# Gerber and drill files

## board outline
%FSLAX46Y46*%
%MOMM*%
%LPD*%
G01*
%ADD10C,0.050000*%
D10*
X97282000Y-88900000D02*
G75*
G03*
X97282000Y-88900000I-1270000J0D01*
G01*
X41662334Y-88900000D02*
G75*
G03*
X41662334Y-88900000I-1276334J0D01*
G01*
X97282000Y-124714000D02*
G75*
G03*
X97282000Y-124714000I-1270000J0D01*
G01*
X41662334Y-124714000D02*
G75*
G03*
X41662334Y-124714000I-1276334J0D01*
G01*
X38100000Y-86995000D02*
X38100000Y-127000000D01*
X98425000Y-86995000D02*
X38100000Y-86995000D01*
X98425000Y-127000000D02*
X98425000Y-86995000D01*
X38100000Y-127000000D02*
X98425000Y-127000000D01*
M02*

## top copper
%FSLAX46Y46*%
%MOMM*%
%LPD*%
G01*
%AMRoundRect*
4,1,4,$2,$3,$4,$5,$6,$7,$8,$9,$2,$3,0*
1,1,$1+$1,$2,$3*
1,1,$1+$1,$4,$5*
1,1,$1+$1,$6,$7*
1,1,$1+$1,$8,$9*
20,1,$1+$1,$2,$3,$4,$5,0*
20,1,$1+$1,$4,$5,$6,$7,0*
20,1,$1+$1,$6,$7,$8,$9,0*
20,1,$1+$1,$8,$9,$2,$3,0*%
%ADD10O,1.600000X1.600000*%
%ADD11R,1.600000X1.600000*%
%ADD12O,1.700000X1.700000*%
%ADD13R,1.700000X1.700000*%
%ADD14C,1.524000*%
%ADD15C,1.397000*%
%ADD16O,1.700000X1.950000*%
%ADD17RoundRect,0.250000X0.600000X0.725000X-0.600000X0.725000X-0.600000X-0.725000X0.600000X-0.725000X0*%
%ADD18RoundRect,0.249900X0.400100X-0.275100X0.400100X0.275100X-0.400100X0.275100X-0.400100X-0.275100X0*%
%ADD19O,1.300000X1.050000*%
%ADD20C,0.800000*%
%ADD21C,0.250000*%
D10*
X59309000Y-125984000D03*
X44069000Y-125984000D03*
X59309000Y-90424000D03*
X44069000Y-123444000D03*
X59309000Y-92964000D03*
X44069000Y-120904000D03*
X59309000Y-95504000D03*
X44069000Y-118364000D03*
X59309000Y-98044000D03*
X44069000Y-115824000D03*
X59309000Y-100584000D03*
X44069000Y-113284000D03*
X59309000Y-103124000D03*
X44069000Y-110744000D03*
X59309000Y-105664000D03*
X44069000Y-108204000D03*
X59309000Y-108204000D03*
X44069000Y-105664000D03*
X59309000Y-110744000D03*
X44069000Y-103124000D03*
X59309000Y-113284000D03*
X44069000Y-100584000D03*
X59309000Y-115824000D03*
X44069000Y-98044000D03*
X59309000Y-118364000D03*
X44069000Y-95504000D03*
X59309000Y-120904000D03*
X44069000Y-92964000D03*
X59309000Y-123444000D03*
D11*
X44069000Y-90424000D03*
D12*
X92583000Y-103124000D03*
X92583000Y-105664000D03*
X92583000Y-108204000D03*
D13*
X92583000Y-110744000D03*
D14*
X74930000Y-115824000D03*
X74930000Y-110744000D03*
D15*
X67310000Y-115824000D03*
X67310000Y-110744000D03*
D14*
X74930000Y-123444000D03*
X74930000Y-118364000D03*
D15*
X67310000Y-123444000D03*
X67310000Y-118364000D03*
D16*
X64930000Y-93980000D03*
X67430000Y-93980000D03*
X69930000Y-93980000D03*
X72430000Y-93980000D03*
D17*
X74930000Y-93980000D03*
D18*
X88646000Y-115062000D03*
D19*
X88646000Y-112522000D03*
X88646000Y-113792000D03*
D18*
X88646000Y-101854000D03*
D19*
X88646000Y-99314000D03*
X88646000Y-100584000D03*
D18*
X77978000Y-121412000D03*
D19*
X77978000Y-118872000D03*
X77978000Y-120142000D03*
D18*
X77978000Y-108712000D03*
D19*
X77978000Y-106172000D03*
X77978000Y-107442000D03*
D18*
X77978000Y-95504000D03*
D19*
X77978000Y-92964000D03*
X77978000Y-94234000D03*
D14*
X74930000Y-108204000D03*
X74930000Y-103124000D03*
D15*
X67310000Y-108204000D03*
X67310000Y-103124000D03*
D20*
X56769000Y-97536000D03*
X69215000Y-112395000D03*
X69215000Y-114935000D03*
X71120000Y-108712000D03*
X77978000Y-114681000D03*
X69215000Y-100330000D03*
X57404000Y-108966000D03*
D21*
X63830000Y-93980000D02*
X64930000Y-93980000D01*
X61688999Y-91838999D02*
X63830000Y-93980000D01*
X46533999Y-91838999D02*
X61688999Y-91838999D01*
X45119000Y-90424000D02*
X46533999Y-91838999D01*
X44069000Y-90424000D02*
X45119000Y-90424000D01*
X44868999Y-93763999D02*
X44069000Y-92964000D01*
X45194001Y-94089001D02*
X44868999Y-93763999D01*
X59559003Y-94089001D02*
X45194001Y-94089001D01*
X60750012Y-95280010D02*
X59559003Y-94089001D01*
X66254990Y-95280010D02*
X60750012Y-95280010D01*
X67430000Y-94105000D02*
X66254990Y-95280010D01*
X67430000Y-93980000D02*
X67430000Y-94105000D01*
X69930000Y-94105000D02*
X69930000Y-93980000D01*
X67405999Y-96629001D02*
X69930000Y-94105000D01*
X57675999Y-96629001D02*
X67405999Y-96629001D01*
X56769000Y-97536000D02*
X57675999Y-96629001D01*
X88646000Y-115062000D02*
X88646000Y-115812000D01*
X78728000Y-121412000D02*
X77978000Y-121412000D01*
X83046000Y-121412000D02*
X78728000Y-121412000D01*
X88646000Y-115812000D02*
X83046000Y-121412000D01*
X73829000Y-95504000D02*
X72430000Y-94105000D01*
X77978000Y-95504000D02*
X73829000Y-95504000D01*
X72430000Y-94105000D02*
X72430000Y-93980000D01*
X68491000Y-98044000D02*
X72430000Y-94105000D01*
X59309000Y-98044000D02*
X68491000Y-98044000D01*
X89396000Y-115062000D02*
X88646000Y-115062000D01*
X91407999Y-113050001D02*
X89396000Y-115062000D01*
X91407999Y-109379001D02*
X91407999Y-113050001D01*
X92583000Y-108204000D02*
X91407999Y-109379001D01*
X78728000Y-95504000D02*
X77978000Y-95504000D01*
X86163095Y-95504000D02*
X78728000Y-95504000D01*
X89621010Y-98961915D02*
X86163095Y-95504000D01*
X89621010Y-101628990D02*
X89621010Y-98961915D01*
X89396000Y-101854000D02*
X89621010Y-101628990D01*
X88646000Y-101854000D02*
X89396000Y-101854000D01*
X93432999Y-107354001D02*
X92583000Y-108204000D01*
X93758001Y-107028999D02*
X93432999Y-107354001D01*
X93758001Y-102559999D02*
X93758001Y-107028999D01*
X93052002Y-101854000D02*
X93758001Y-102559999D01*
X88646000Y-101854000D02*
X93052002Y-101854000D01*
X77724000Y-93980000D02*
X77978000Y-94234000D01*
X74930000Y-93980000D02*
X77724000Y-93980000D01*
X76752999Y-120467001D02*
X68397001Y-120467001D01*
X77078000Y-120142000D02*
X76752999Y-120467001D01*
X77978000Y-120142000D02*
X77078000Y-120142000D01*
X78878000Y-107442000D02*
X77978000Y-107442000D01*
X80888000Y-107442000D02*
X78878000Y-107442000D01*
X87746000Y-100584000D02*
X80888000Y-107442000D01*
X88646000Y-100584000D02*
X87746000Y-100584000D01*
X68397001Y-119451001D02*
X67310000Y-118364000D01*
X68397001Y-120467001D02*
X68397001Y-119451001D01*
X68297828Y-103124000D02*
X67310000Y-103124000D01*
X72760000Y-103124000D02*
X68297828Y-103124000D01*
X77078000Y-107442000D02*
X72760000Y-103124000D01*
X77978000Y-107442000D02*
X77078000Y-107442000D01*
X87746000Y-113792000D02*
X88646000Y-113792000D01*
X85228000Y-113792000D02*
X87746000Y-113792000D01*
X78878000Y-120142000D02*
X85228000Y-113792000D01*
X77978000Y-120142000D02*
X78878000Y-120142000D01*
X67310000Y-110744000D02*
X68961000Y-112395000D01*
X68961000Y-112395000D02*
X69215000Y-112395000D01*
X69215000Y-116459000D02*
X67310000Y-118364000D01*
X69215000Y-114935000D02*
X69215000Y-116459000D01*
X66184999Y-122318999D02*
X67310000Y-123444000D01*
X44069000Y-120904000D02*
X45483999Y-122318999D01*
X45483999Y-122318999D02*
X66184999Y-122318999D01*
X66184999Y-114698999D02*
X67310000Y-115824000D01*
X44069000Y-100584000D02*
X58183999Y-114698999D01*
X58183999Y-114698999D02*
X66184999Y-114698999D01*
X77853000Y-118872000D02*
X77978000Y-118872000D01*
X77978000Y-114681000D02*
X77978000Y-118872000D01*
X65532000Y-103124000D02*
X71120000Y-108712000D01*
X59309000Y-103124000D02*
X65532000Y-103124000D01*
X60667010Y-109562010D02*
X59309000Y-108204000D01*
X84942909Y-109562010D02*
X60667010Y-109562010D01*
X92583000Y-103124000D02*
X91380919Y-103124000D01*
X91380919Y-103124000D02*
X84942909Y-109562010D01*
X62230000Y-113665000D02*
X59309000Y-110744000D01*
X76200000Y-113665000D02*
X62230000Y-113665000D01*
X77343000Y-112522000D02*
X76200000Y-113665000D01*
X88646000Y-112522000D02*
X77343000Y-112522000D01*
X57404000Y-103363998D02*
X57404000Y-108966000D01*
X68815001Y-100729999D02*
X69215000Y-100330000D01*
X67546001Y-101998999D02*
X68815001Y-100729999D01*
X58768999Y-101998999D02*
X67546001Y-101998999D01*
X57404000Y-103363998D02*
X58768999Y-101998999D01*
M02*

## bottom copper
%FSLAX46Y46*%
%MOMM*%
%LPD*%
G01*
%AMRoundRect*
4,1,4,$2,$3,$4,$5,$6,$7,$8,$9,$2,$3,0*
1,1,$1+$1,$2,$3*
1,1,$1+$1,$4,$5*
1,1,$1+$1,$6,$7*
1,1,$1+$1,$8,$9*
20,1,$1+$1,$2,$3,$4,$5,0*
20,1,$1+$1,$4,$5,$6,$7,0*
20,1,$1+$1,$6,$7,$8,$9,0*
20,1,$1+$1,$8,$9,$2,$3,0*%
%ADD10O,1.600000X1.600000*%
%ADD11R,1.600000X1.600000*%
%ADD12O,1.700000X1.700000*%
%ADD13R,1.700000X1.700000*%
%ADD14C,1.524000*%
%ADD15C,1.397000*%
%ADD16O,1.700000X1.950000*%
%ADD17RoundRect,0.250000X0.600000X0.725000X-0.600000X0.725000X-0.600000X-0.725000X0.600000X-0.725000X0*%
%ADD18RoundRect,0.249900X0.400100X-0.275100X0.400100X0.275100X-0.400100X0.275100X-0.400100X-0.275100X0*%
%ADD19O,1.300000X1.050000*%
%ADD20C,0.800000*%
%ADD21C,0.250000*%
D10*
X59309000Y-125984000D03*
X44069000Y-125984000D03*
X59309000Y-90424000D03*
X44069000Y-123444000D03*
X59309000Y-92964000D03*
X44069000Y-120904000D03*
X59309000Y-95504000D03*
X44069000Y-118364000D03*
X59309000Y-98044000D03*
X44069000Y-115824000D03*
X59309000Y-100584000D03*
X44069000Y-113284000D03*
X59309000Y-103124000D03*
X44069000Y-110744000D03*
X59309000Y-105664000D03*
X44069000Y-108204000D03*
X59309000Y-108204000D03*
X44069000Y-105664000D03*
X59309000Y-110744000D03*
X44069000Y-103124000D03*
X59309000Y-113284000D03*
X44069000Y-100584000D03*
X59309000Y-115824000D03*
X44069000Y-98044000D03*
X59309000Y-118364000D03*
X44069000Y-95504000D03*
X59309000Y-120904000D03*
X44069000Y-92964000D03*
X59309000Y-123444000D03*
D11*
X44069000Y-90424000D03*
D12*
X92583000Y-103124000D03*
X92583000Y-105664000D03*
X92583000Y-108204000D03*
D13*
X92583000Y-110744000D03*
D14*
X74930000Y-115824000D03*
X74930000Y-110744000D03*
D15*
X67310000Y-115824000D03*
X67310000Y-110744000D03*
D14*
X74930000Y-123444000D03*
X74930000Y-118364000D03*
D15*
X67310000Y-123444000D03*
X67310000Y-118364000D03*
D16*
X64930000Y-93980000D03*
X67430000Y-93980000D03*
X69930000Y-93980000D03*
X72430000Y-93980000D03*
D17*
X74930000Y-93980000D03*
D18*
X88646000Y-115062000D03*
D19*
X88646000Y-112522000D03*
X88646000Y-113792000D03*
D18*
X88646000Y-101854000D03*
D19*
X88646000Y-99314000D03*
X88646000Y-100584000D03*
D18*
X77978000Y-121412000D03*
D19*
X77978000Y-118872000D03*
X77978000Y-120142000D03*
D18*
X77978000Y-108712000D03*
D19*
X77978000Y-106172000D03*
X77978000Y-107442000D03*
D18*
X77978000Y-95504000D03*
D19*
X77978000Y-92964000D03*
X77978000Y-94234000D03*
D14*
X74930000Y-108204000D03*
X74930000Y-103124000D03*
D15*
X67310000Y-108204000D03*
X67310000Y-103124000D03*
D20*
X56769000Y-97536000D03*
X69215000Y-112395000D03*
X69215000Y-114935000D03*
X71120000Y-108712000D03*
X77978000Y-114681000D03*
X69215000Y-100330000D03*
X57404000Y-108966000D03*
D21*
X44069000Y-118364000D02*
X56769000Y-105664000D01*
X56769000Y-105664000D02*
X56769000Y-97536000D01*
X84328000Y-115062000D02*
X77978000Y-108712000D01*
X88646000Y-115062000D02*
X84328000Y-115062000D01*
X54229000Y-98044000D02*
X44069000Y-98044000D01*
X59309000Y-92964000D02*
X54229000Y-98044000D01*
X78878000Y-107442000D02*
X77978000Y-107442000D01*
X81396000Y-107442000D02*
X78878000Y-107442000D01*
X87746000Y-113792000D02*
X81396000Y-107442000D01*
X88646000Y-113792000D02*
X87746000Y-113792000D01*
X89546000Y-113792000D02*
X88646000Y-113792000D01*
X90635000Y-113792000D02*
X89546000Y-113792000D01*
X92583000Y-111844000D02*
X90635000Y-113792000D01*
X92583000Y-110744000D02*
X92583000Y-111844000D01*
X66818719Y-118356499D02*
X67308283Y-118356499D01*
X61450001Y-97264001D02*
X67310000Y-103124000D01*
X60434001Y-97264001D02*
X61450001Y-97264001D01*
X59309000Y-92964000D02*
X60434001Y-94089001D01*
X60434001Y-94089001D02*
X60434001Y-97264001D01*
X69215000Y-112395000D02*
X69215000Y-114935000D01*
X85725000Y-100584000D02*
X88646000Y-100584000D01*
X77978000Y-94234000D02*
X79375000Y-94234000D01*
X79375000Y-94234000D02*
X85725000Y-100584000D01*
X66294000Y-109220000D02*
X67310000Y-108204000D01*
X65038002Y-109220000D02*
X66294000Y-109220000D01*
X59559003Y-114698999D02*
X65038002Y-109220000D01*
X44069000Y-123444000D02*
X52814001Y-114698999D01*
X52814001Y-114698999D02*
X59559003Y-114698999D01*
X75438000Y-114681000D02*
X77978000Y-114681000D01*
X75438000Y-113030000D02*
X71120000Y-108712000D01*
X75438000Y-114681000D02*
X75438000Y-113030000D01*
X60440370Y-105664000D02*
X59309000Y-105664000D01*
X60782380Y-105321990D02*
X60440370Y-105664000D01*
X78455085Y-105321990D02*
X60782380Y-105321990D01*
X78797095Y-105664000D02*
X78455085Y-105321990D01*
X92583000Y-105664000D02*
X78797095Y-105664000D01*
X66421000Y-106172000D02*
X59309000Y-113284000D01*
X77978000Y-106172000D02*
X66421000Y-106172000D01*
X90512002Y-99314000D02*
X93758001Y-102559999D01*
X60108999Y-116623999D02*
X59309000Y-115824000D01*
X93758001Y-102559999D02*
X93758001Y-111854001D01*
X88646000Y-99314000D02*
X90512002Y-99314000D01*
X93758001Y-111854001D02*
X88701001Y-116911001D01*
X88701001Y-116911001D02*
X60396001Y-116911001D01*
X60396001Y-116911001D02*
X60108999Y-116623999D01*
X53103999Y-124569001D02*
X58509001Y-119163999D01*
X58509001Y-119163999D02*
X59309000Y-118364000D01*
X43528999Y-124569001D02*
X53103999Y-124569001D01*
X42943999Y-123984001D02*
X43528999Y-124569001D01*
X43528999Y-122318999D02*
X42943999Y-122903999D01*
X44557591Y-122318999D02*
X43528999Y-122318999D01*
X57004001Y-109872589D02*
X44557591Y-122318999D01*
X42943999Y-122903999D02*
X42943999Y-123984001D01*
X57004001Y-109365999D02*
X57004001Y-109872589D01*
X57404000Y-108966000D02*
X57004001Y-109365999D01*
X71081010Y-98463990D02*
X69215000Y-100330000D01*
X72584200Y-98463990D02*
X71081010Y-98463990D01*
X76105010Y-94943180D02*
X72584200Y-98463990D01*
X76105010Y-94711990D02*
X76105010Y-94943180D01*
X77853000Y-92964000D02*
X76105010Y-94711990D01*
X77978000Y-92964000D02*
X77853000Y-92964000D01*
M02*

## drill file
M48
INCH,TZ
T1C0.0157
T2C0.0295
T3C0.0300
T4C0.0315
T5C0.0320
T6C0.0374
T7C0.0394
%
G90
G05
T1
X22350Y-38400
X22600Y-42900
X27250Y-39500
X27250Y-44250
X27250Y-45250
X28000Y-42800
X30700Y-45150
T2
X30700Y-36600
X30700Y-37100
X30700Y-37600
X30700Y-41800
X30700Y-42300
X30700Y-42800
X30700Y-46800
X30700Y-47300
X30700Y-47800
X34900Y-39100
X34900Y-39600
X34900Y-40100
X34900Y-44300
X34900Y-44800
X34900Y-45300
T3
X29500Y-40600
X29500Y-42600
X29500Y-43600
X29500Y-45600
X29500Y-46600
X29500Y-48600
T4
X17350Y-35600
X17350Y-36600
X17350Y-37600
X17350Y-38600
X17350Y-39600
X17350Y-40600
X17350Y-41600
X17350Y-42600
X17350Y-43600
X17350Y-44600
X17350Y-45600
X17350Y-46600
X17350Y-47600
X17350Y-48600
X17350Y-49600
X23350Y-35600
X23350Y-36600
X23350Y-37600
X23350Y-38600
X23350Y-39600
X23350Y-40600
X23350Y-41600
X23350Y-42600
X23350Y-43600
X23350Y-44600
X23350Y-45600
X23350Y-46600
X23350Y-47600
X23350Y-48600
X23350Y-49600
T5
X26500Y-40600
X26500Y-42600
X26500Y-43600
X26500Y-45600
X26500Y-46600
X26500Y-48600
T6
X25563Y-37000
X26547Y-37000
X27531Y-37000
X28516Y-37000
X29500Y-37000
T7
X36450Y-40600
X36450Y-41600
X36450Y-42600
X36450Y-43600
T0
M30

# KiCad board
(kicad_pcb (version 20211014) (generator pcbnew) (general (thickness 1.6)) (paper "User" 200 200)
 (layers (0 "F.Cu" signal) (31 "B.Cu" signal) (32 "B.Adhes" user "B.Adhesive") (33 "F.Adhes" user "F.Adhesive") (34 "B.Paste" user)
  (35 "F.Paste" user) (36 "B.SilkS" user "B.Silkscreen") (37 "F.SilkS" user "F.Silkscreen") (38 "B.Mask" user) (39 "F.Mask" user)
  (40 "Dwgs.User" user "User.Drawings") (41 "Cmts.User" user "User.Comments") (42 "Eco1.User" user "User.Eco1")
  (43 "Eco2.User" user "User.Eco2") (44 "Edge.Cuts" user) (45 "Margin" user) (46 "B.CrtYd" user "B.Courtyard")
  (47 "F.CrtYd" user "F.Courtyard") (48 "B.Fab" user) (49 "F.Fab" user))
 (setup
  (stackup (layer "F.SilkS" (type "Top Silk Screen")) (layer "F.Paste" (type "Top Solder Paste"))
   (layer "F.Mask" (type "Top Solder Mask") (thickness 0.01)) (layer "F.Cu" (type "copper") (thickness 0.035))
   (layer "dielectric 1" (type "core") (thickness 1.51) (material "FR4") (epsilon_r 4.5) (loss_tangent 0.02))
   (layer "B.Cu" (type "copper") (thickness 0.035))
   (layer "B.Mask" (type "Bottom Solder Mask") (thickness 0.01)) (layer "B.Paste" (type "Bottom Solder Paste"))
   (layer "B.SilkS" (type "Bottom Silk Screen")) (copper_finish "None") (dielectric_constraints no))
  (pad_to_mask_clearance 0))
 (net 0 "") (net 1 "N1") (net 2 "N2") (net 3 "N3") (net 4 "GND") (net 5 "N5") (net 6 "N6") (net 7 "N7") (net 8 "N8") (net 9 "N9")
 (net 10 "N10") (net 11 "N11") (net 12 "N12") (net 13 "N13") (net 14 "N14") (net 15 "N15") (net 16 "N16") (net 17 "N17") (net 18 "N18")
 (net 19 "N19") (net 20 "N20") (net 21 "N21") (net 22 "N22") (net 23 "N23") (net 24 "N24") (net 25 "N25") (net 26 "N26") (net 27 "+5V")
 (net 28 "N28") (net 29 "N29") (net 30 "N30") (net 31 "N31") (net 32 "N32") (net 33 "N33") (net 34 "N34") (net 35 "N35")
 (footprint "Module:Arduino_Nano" (layer "F.Cu") (at 44.069 90.424)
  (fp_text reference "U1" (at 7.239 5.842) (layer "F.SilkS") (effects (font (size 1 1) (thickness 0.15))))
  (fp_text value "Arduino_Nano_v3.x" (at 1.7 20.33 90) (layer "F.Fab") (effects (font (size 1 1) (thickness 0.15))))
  (pad "1" thru_hole rect locked (at 0 0) (size 1.6 1.6) (drill 0.8) (layers *.Cu *.Mask) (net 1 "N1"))
  (pad "2" thru_hole oval locked (at 0 2.54) (size 1.6 1.6) (drill 0.8) (layers *.Cu *.Mask) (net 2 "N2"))
  (pad "3" thru_hole oval locked (at 0 5.08) (size 1.6 1.6) (drill 0.8) (layers *.Cu *.Mask) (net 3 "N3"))
  (pad "4" thru_hole oval locked (at 0 7.62) (size 1.6 1.6) (drill 0.8) (layers *.Cu *.Mask) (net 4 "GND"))
  (pad "5" thru_hole oval locked (at 0 10.16) (size 1.6 1.6) (drill 0.8) (layers *.Cu *.Mask) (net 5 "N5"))
  (pad "6" thru_hole oval locked (at 0 12.7) (size 1.6 1.6) (drill 0.8) (layers *.Cu *.Mask) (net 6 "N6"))
  (pad "7" thru_hole oval locked (at 0 15.24) (size 1.6 1.6) (drill 0.8) (layers *.Cu *.Mask) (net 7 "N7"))
  (pad "8" thru_hole oval locked (at 0 17.78) (size 1.6 1.6) (drill 0.8) (layers *.Cu *.Mask) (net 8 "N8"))
  (pad "9" thru_hole oval locked (at 0 20.32) (size 1.6 1.6) (drill 0.8) (layers *.Cu *.Mask) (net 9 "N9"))
  (pad "10" thru_hole oval locked (at 0 22.86) (size 1.6 1.6) (drill 0.8) (layers *.Cu *.Mask) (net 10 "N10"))
  (pad "11" thru_hole oval locked (at 0 25.4) (size 1.6 1.6) (drill 0.8) (layers *.Cu *.Mask) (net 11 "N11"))
  (pad "12" thru_hole oval locked (at 0 27.94) (size 1.6 1.6) (drill 0.8) (layers *.Cu *.Mask) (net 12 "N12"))
  (pad "13" thru_hole oval locked (at 0 30.48) (size 1.6 1.6) (drill 0.8) (layers *.Cu *.Mask) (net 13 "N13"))
  (pad "14" thru_hole oval locked (at 0 33.02) (size 1.6 1.6) (drill 0.8) (layers *.Cu *.Mask) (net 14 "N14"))
  (pad "15" thru_hole oval locked (at 0 35.56) (size 1.6 1.6) (drill 0.8) (layers *.Cu *.Mask) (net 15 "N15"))
  (pad "16" thru_hole oval locked (at 15.24 35.56) (size 1.6 1.6) (drill 0.8) (layers *.Cu *.Mask) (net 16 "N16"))
  (pad "17" thru_hole oval locked (at 15.24 33.02) (size 1.6 1.6) (drill 0.8) (layers *.Cu *.Mask) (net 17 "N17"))
  (pad "18" thru_hole oval locked (at 15.24 30.48) (size 1.6 1.6) (drill 0.8) (layers *.Cu *.Mask) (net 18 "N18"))
  (pad "19" thru_hole oval locked (at 15.24 27.94) (size 1.6 1.6) (drill 0.8) (layers *.Cu *.Mask) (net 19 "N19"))
  (pad "20" thru_hole oval locked (at 15.24 25.4) (size 1.6 1.6) (drill 0.8) (layers *.Cu *.Mask) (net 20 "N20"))
  (pad "21" thru_hole oval locked (at 15.24 22.86) (size 1.6 1.6) (drill 0.8) (layers *.Cu *.Mask) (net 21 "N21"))
  (pad "22" thru_hole oval locked (at 15.24 20.32) (size 1.6 1.6) (drill 0.8) (layers *.Cu *.Mask) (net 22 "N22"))
  (pad "23" thru_hole oval locked (at 15.24 17.78) (size 1.6 1.6) (drill 0.8) (layers *.Cu *.Mask) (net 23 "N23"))
  (pad "24" thru_hole oval locked (at 15.24 15.24) (size 1.6 1.6) (drill 0.8) (layers *.Cu *.Mask) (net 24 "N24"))
  (pad "25" thru_hole oval locked (at 15.24 12.7) (size 1.6 1.6) (drill 0.8) (layers *.Cu *.Mask) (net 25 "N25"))
  (pad "26" thru_hole oval locked (at 15.24 10.16) (size 1.6 1.6) (drill 0.8) (layers *.Cu *.Mask) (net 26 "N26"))
  (pad "27" thru_hole oval locked (at 15.24 7.62) (size 1.6 1.6) (drill 0.8) (layers *.Cu *.Mask) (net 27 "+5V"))
  (pad "28" thru_hole oval locked (at 15.24 5.08) (size 1.6 1.6) (drill 0.8) (layers *.Cu *.Mask) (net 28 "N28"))
  (pad "29" thru_hole oval locked (at 15.24 2.54) (size 1.6 1.6) (drill 0.8) (layers *.Cu *.Mask) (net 4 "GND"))
  (pad "30" thru_hole oval locked (at 15.24 0) (size 1.6 1.6) (drill 0.8) (layers *.Cu *.Mask) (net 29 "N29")))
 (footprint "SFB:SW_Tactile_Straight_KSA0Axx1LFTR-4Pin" (layer "F.Cu") (at 67.31 103.124)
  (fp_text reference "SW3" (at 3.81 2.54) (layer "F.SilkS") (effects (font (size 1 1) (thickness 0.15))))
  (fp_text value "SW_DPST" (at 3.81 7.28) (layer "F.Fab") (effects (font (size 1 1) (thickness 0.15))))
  (pad "1" thru_hole circle locked (at 0 0) (size 1.397 1.397) (drill 0.8128) (layers *.Cu *.Mask) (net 4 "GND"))
  (pad "2" thru_hole circle locked (at 0 5.08) (size 1.397 1.397) (drill 0.8128) (layers *.Cu *.Mask) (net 14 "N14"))
  (pad "3" thru_hole circle locked (at 7.62 0) (size 1.524 1.524) (drill 0.762) (layers *.Cu *.Mask) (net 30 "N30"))
  (pad "4" thru_hole circle locked (at 7.62 5.08) (size 1.524 1.524) (drill 0.762) (layers *.Cu *.Mask) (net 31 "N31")))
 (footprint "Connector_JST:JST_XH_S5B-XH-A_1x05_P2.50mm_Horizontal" (layer "F.Cu") (at 74.93 93.98 180)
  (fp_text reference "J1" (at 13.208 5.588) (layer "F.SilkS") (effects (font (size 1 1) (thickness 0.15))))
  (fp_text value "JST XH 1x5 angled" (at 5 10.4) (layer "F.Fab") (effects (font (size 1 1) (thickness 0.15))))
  (pad "1" thru_hole roundrect locked (at 0 0 180) (size 1.7 1.95) (drill 0.95) (layers *.Cu *.Mask) (roundrect_rratio 0.1470588235)
   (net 4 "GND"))
  (pad "2" thru_hole oval locked (at 2.5 0 180) (size 1.7 1.95) (drill 0.95) (layers *.Cu *.Mask) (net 27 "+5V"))
  (pad "3" thru_hole oval locked (at 5 0 180) (size 1.7 1.95) (drill 0.95) (layers *.Cu *.Mask) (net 12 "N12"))
  (pad "4" thru_hole oval locked (at 7.5 0 180) (size 1.7 1.95) (drill 0.95) (layers *.Cu *.Mask) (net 2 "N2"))
  (pad "5" thru_hole oval locked (at 10 0 180) (size 1.7 1.95) (drill 0.95) (layers *.Cu *.Mask) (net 1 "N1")))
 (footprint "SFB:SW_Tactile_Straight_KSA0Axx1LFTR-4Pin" (layer "F.Cu") (at 67.31 118.364)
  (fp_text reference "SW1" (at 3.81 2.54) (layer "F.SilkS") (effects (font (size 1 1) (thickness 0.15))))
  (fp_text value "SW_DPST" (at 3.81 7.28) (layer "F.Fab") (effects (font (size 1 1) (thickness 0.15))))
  (pad "1" thru_hole circle locked (at 0 0) (size 1.397 1.397) (drill 0.8128) (layers *.Cu *.Mask) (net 4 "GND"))
  (pad "2" thru_hole circle locked (at 0 5.08) (size 1.397 1.397) (drill 0.8128) (layers *.Cu *.Mask) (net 13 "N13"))
  (pad "3" thru_hole circle locked (at 7.62 0) (size 1.524 1.524) (drill 0.762) (layers *.Cu *.Mask) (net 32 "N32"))
  (pad "4" thru_hole circle locked (at 7.62 5.08) (size 1.524 1.524) (drill 0.762) (layers *.Cu *.Mask) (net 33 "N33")))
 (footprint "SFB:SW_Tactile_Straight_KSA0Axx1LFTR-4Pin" (layer "F.Cu") (at 67.31 110.744)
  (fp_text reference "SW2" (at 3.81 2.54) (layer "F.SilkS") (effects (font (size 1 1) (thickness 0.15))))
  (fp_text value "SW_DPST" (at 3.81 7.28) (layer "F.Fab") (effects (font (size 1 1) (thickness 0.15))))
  (pad "1" thru_hole circle locked (at 0 0) (size 1.397 1.397) (drill 0.8128) (layers *.Cu *.Mask) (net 4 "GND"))
  (pad "2" thru_hole circle locked (at 0 5.08) (size 1.397 1.397) (drill 0.8128) (layers *.Cu *.Mask) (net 5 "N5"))
  (pad "3" thru_hole circle locked (at 7.62 0) (size 1.524 1.524) (drill 0.762) (layers *.Cu *.Mask) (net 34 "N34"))
  (pad "4" thru_hole circle locked (at 7.62 5.08) (size 1.524 1.524) (drill 0.762) (layers *.Cu *.Mask) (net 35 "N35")))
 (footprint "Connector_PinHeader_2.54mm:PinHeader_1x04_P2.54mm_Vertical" (layer "F.Cu") (at 92.583 110.744 180)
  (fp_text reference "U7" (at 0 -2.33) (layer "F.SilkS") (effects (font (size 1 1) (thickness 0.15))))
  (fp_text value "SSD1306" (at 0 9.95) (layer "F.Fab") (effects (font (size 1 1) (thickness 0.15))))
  (pad "1" thru_hole rect locked (at 0 0 180) (size 1.7 1.7) (drill 1) (layers *.Cu *.Mask) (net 4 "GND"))
  (pad "2" thru_hole oval locked (at 0 2.54 180) (size 1.7 1.7) (drill 1) (layers *.Cu *.Mask) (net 27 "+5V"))
  (pad "3" thru_hole oval locked (at 0 5.08 180) (size 1.7 1.7) (drill 1) (layers *.Cu *.Mask) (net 24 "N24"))
  (pad "4" thru_hole oval locked (at 0 7.62 180) (size 1.7 1.7) (drill 1) (layers *.Cu *.Mask) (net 23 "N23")))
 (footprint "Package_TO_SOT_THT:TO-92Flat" (layer "B.Cu") (at 77.978 121.412 90)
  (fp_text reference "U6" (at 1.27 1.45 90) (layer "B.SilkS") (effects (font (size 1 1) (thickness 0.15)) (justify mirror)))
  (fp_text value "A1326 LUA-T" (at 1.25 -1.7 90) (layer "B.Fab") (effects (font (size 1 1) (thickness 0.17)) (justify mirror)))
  (pad "1" thru_hole roundrect locked (at 0 0 90) (size 1.05 1.3) (drill 0.75) (layers *.Cu *.Mask) (roundrect_rratio 0.238) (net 27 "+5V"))
  (pad "2" thru_hole oval locked (at 1.27 0 90) (size 1.05 1.3) (drill 0.75) (layers *.Cu *.Mask) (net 4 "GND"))
  (pad "3" thru_hole oval locked (at 2.54 0 90) (size 1.05 1.3) (drill 0.75) (layers *.Cu *.Mask) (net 25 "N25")))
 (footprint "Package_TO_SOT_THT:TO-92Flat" (layer "B.Cu") (at 88.646 101.854 90)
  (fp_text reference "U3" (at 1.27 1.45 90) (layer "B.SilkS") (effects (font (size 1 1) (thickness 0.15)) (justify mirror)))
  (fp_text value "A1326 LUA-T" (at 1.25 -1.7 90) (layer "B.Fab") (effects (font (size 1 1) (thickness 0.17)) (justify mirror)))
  (pad "1" thru_hole roundrect locked (at 0 0 90) (size 1.05 1.3) (drill 0.75) (layers *.Cu *.Mask) (roundrect_rratio 0.238) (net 27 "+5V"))
  (pad "2" thru_hole oval locked (at 1.27 0 90) (size 1.05 1.3) (drill 0.75) (layers *.Cu *.Mask) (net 4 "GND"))
  (pad "3" thru_hole oval locked (at 2.54 0 90) (size 1.05 1.3) (drill 0.75) (layers *.Cu *.Mask) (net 20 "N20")))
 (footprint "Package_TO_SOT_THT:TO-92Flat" (layer "B.Cu") (at 88.646 115.062 90)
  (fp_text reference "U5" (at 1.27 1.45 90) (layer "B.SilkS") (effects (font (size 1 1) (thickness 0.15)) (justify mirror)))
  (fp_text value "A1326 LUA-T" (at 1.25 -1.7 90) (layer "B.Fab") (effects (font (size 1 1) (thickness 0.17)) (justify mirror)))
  (pad "1" thru_hole roundrect locked (at 0 0 90) (size 1.05 1.3) (drill 0.75) (layers *.Cu *.Mask) (roundrect_rratio 0.238) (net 27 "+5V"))
  (pad "2" thru_hole oval locked (at 1.27 0 90) (size 1.05 1.3) (drill 0.75) (layers *.Cu *.Mask) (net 4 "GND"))
  (pad "3" thru_hole oval locked (at 2.54 0 90) (size 1.05 1.3) (drill 0.75) (layers *.Cu *.Mask) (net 22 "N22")))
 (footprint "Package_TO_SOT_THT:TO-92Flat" (layer "B.Cu") (at 77.978 108.712 90)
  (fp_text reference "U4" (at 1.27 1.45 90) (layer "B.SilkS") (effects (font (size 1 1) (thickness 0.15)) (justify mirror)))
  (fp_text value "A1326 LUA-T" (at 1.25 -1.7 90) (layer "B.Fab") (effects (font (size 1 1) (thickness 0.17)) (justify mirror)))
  (pad "1" thru_hole roundrect locked (at 0 0 90) (size 1.05 1.3) (drill 0.75) (layers *.Cu *.Mask) (roundrect_rratio 0.238) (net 27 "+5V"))
  (pad "2" thru_hole oval locked (at 1.27 0 90) (size 1.05 1.3) (drill 0.75) (layers *.Cu *.Mask) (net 4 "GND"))
  (pad "3" thru_hole oval locked (at 2.54 0 90) (size 1.05 1.3) (drill 0.75) (layers *.Cu *.Mask) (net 21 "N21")))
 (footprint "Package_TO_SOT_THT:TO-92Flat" (layer "B.Cu") (at 77.978 95.504 90)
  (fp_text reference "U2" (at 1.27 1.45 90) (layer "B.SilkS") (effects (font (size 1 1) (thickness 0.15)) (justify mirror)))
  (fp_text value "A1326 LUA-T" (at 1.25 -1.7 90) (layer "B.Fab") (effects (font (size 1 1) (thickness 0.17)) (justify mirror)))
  (pad "1" thru_hole roundrect locked (at 0 0 90) (size 1.05 1.3) (drill 0.75) (layers *.Cu *.Mask) (roundrect_rratio 0.238) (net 27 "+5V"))
  (pad "2" thru_hole oval locked (at 1.27 0 90) (size 1.05 1.3) (drill 0.75) (layers *.Cu *.Mask) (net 4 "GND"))
  (pad "3" thru_hole oval locked (at 2.54 0 90) (size 1.05 1.3) (drill 0.75) (layers *.Cu *.Mask) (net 19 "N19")))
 (gr_line (start 98.425 127) (end 98.425 86.995) (layer "Edge.Cuts") (width 0.05))
 (gr_line (start 98.425 86.995) (end 38.1 86.995) (layer "Edge.Cuts") (width 0.05))
 (gr_line (start 38.1 86.995) (end 38.1 127) (layer "Edge.Cuts") (width 0.05))
 (gr_line (start 38.1 127) (end 98.425 127) (layer "Edge.Cuts") (width 0.05))
 (gr_circle (center 40.386 124.714) (end 41.656 124.841) (layer "Edge.Cuts") (width 0.05) (fill none))
 (gr_circle (center 96.012 88.9) (end 97.282 88.9) (layer "Edge.Cuts") (width 0.05) (fill none))
 (gr_circle (center 96.012 124.714) (end 97.282 124.714) (layer "Edge.Cuts") (width 0.05) (fill none))
 (gr_circle (center 40.386 88.9) (end 41.656 89.027) (layer "Edge.Cuts") (width 0.05) (fill none))
 (segment (start 61.688999 91.838999) (end 63.83 93.98) (width 0.25) (layer "F.Cu") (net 1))
 (segment (start 46.533999 91.838999) (end 61.688999 91.838999) (width 0.25) (layer "F.Cu") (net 1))
 (segment (start 63.83 93.98) (end 64.93 93.98) (width 0.25) (layer "F.Cu") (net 1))
 (segment (start 44.069 90.424) (end 45.119 90.424) (width 0.25) (layer "F.Cu") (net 1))
 (segment (start 45.119 90.424) (end 46.533999 91.838999) (width 0.25) (layer "F.Cu") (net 1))
 (segment (start 67.43 94.105) (end 66.25499 95.28001) (width 0.25) (layer "F.Cu") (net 2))
 (segment (start 67.43 93.98) (end 67.43 94.105) (width 0.25) (layer "F.Cu") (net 2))
 (segment (start 66.25499 95.28001) (end 60.750012 95.28001) (width 0.25) (layer "F.Cu") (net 2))
 (segment (start 60.750012 95.28001) (end 59.559003 94.089001) (width 0.25) (layer "F.Cu") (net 2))
 (segment (start 45.194001 94.089001) (end 44.868999 93.763999) (width 0.25) (layer "F.Cu") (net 2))
 (segment (start 44.868999 93.763999) (end 44.069 92.964) (width 0.25) (layer "F.Cu") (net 2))
 (segment (start 59.559003 94.089001) (end 45.194001 94.089001) (width 0.25) (layer "F.Cu") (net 2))
 (segment (start 56.769 97.536) (end 57.675999 96.629001) (width 0.25) (layer "F.Cu") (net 12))
 (segment (start 67.405999 96.629001) (end 69.93 94.105) (width 0.25) (layer "F.Cu") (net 12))
 (segment (start 57.675999 96.629001) (end 67.405999 96.629001) (width 0.25) (layer "F.Cu") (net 12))
 (segment (start 69.93 94.105) (end 69.93 93.98) (width 0.25) (layer "F.Cu") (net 12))
 (via (at 56.769 97.536) (size 0.8) (drill 0.4) (layers "F.Cu" "B.Cu") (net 12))
 (segment (start 44.069 118.364) (end 56.769 105.664) (width 0.25) (layer "B.Cu") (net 12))
 (segment (start 56.769 105.664) (end 56.769 97.536) (width 0.25) (layer "B.Cu") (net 12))
 (segment (start 93.432999 107.354001) (end 92.583 108.204) (width 0.25) (layer "F.Cu") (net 27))
 (segment (start 89.396 115.062) (end 88.646 115.062) (width 0.25) (layer "F.Cu") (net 27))
 (segment (start 89.62101 98.961915) (end 86.163095 95.504) (width 0.25) (layer "F.Cu") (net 27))
 (segment (start 73.829 95.504) (end 72.43 94.105) (width 0.25) (layer "F.Cu") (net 27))
 (segment (start 86.163095 95.504) (end 78.728 95.504) (width 0.25) (layer "F.Cu") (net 27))
 (segment (start 92.583 108.204) (end 91.407999 109.379001) (width 0.25) (layer "F.Cu") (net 27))
 (segment (start 89.62101 101.62899) (end 89.62101 98.961915) (width 0.25) (layer "F.Cu") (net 27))
 (segment (start 93.758001 107.028999) (end 93.432999 107.354001) (width 0.25) (layer "F.Cu") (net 27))
 (segment (start 78.728 121.412) (end 77.978 121.412) (width 0.25) (layer "F.Cu") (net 27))
 (segment (start 89.396 101.854) (end 89.62101 101.62899) (width 0.25) (layer "F.Cu") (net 27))
 (segment (start 88.646 101.854) (end 93.052002 101.854) (width 0.25) (layer "F.Cu") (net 27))
 (segment (start 68.491 98.044) (end 72.43 94.105) (width 0.25) (layer "F.Cu") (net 27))
 (segment (start 91.407999 109.379001) (end 91.407999 113.050001) (width 0.25) (layer "F.Cu") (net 27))
 (segment (start 91.407999 113.050001) (end 89.396 115.062) (width 0.25) (layer "F.Cu") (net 27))
 (segment (start 72.43 94.105) (end 72.43 93.98) (width 0.25) (layer "F.Cu") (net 27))
 (segment (start 88.646 115.062) (end 88.646 115.812) (width 0.25) (layer "F.Cu") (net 27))
 (segment (start 83.046 121.412) (end 78.728 121.412) (width 0.25) (layer "F.Cu") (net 27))
 (segment (start 93.758001 102.559999) (end 93.758001 107.028999) (width 0.25) (layer "F.Cu") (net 27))
 (segment (start 88.646 115.812) (end 83.046 121.412) (width 0.25) (layer "F.Cu") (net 27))
 (segment (start 78.728 95.504) (end 77.978 95.504) (width 0.25) (layer "F.Cu") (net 27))
 (segment (start 77.978 95.504) (end 73.829 95.504) (width 0.25) (layer "F.Cu") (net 27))
 (segment (start 88.646 101.854) (end 89.396 101.854) (width 0.25) (layer "F.Cu") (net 27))
 (segment (start 93.052002 101.854) (end 93.758001 102.559999) (width 0.25) (layer "F.Cu") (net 27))
 (segment (start 59.309 98.044) (end 68.491 98.044) (width 0.25) (layer "F.Cu") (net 27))
 (segment (start 84.328 115.062) (end 77.978 108.712) (width 0.25) (layer "B.Cu") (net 27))
 (segment (start 88.646 115.062) (end 84.328 115.062) (width 0.25) (layer "B.Cu") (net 27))
 (segment (start 88.646 100.584) (end 87.746 100.584) (width 0.25) (layer "F.Cu") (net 4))
 (segment (start 85.228 113.792) (end 87.746 113.792) (width 0.25) (layer "F.Cu") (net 4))
 (segment (start 77.078 120.142) (end 76.752999 120.467001) (width 0.25) (layer "F.Cu") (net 4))
 (segment (start 69.215 114.935) (end 69.215 116.459) (width 0.25) (layer "F.Cu") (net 4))
 (segment (start 77.078 107.442) (end 72.76 103.124) (width 0.25) (layer "F.Cu") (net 4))
 (segment (start 77.978 120.142) (end 77.078 120.142) (width 0.25) (layer "F.Cu") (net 4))
 (segment (start 68.397001 119.451001) (end 67.31 118.364) (width 0.25) (layer "F.Cu") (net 4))
 (segment (start 80.888 107.442) (end 78.878 107.442) (width 0.25) (layer "F.Cu") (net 4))
 (segment (start 76.752999 120.467001) (end 68.397001 120.467001) (width 0.25) (layer "F.Cu") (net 4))
 (segment (start 69.215 116.459) (end 67.31 118.364) (width 0.25) (layer "F.Cu") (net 4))
 (segment (start 74.93 93.98) (end 77.724 93.98) (width 0.25) (layer "F.Cu") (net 4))
 (segment (start 72.76 103.124) (end 68.297828 103.124) (width 0.25) (layer "F.Cu") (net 4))
 (segment (start 67.31 110.744) (end 68.961 112.395) (width 0.25) (layer "F.Cu") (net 4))
 (segment (start 78.878 107.442) (end 77.978 107.442) (width 0.25) (layer "F.Cu") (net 4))
 (segment (start 87.746 100.584) (end 80.888 107.442) (width 0.25) (layer "F.Cu") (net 4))
 (segment (start 77.978 120.142) (end 78.878 120.142) (width 0.25) (layer "F.Cu") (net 4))
 (segment (start 77.978 107.442) (end 77.078 107.442) (width 0.25) (layer "F.Cu") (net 4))
 (segment (start 87.746 113.792) (end 88.646 113.792) (width 0.25) (layer "F.Cu") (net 4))
 (segment (start 68.297828 103.124) (end 67.31 103.124) (width 0.25) (layer "F.Cu") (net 4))
 (segment (start 77.724 93.98) (end 77.978 94.234) (width 0.25) (layer "F.Cu") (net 4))
 (segment (start 78.878 120.142) (end 85.228 113.792) (width 0.25) (layer "F.Cu") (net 4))
 (segment (start 68.961 112.395) (end 69.215 112.395) (width 0.25) (layer "F.Cu") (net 4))
 (segment (start 68.397001 120.467001) (end 68.397001 119.451001) (width 0.25) (layer "F.Cu") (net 4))
 (via (at 69.215 114.935) (size 0.8) (drill 0.4) (layers "F.Cu" "B.Cu") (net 4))
 (via (at 69.215 112.395) (size 0.8) (drill 0.4) (layers "F.Cu" "B.Cu") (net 4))
 (segment (start 85.725 100.584) (end 88.646 100.584) (width 0.25) (layer "B.Cu") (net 4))
 (segment (start 78.878 107.442) (end 77.978 107.442) (width 0.25) (layer "B.Cu") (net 4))
 (segment (start 59.309 92.964) (end 54.229 98.044) (width 0.25) (layer "B.Cu") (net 4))
 (segment (start 59.309 92.964) (end 60.434001 94.089001) (width 0.25) (layer "B.Cu") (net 4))
 (segment (start 61.450001 97.264001) (end 67.31 103.124) (width 0.25) (layer "B.Cu") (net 4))
 (segment (start 60.434001 97.264001) (end 61.450001 97.264001) (width 0.25) (layer "B.Cu") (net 4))
 (segment (start 87.746 113.792) (end 81.396 107.442) (width 0.25) (layer "B.Cu") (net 4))
 (segment (start 54.229 98.044) (end 44.069 98.044) (width 0.25) (layer "B.Cu") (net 4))
 (segment (start 77.978 94.234) (end 79.375 94.234) (width 0.25) (layer "B.Cu") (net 4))
 (segment (start 81.396 107.442) (end 78.878 107.442) (width 0.25) (layer "B.Cu") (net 4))
 (segment (start 88.646 113.792) (end 87.746 113.792) (width 0.25) (layer "B.Cu") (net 4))
 (segment (start 92.583 111.844) (end 90.635 113.792) (width 0.25) (layer "B.Cu") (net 4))
 (segment (start 92.583 110.744) (end 92.583 111.844) (width 0.25) (layer "B.Cu") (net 4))
 (segment (start 66.818719 118.356499) (end 67.308283 118.356499) (width 0.25) (layer "B.Cu") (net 4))
 (segment (start 79.375 94.234) (end 85.725 100.584) (width 0.25) (layer "B.Cu") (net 4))
 (segment (start 60.434001 94.089001) (end 60.434001 97.264001) (width 0.25) (layer "B.Cu") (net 4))
 (segment (start 89.546 113.792) (end 88.646 113.792) (width 0.25) (layer "B.Cu") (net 4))
 (segment (start 90.635 113.792) (end 89.546 113.792) (width 0.25) (layer "B.Cu") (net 4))
 (segment (start 69.215 112.395) (end 69.215 114.935) (width 0.25) (layer "B.Cu") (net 4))
 (segment (start 44.069 120.904) (end 45.483999 122.318999) (width 0.25) (layer "F.Cu") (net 13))
 (segment (start 66.184999 122.318999) (end 67.31 123.444) (width 0.25) (layer "F.Cu") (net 13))
 (segment (start 45.483999 122.318999) (end 66.184999 122.318999) (width 0.25) (layer "F.Cu") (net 13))
 (segment (start 44.069 100.584) (end 58.183999 114.698999) (width 0.25) (layer "F.Cu") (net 5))
 (segment (start 66.184999 114.698999) (end 67.31 115.824) (width 0.25) (layer "F.Cu") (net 5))
 (segment (start 58.183999 114.698999) (end 66.184999 114.698999) (width 0.25) (layer "F.Cu") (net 5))
 (segment (start 44.069 123.444) (end 52.814001 114.698999) (width 0.25) (layer "B.Cu") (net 14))
 (segment (start 52.814001 114.698999) (end 59.559003 114.698999) (width 0.25) (layer "B.Cu") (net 14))
 (segment (start 66.294 109.22) (end 67.31 108.204) (width 0.25) (layer "B.Cu") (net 14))
 (segment (start 65.038002 109.22) (end 66.294 109.22) (width 0.25) (layer "B.Cu") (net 14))
 (segment (start 59.559003 114.698999) (end 65.038002 109.22) (width 0.25) (layer "B.Cu") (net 14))
 (segment (start 59.309 103.124) (end 65.532 103.124) (width 0.25) (layer "F.Cu") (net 25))
 (segment (start 77.853 118.872) (end 77.978 118.872) (width 0.25) (layer "F.Cu") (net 25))
 (segment (start 77.978 114.681) (end 77.978 118.872) (width 0.25) (layer "F.Cu") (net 25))
 (segment (start 65.532 103.124) (end 71.12 108.712) (width 0.25) (layer "F.Cu") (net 25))
 (via (at 71.12 108.712) (size 0.8) (drill 0.4) (layers "F.Cu" "B.Cu") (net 25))
 (via (at 77.978 114.681) (size 0.8) (drill 0.4) (layers "F.Cu" "B.Cu") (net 25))
 (segment (start 75.438 114.681) (end 77.978 114.681) (width 0.25) (layer "B.Cu") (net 25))
 (segment (start 75.438 113.03) (end 71.12 108.712) (width 0.25) (layer "B.Cu") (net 25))
 (segment (start 75.438 114.681) (end 75.438 113.03) (width 0.25) (layer "B.Cu") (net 25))
 (segment (start 92.583 105.664) (end 78.797095 105.664) (width 0.25) (layer "B.Cu") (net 24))
 (segment (start 78.797095 105.664) (end 78.455085 105.32199) (width 0.25) (layer "B.Cu") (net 24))
 (segment (start 78.455085 105.32199) (end 60.78238 105.32199) (width 0.25) (layer "B.Cu") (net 24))
 (segment (start 60.78238 105.32199) (end 60.44037 105.664) (width 0.25) (layer "B.Cu") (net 24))
 (segment (start 60.44037 105.664) (end 59.309 105.664) (width 0.25) (layer "B.Cu") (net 24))
 (segment (start 84.942909 109.56201) (end 60.66701 109.56201) (width 0.25) (layer "F.Cu") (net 23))
 (segment (start 91.380919 103.124) (end 84.942909 109.56201) (width 0.25) (layer "F.Cu") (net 23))
 (segment (start 60.66701 109.56201) (end 59.309 108.204) (width 0.25) (layer "F.Cu") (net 23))
 (segment (start 92.583 103.124) (end 91.380919 103.124) (width 0.25) (layer "F.Cu") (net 23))
 (segment (start 62.23 113.665) (end 59.309 110.744) (width 0.25) (layer "F.Cu") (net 22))
 (segment (start 76.2 113.665) (end 62.23 113.665) (width 0.25) (layer "F.Cu") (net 22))
 (segment (start 77.343 112.522) (end 76.2 113.665) (width 0.25) (layer "F.Cu") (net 22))
 (segment (start 88.646 112.522) (end 77.343 112.522) (width 0.25) (layer "F.Cu") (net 22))
 (segment (start 77.978 106.172) (end 66.421 106.172) (width 0.25) (layer "B.Cu") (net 21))
 (segment (start 66.421 106.172) (end 59.309 113.284) (width 0.25) (layer "B.Cu") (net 21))
 (segment (start 60.108999 116.623999) (end 59.309 115.824) (width 0.25) (layer "B.Cu") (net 20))
 (segment (start 60.396001 116.911001) (end 60.108999 116.623999) (width 0.25) (layer "B.Cu") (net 20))
 (segment (start 93.758001 111.854001) (end 88.701001 116.911001) (width 0.25) (layer "B.Cu") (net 20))
 (segment (start 90.512002 99.314) (end 93.758001 102.559999) (width 0.25) (layer "B.Cu") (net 20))
 (segment (start 88.646 99.314) (end 90.512002 99.314) (width 0.25) (layer "B.Cu") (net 20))
 (segment (start 88.701001 116.911001) (end 60.396001 116.911001) (width 0.25) (layer "B.Cu") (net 20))
 (segment (start 93.758001 102.559999) (end 93.758001 111.854001) (width 0.25) (layer "B.Cu") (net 20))
 (segment (start 68.815001 100.729999) (end 69.215 100.33) (width 0.25) (layer "F.Cu") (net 19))
 (segment (start 57.404 103.363998) (end 57.404 108.966) (width 0.25) (layer "F.Cu") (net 19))
 (segment (start 58.768999 101.998999) (end 67.546001 101.998999) (width 0.25) (layer "F.Cu") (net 19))
 (segment (start 57.404 103.363998) (end 58.768999 101.998999) (width 0.25) (layer "F.Cu") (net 19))
 (segment (start 67.546001 101.998999) (end 68.815001 100.729999) (width 0.25) (layer "F.Cu") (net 19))
 (via (at 69.215 100.33) (size 0.8) (drill 0.4) (layers "F.Cu" "B.Cu") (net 19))
 (via (at 57.404 108.966) (size 0.8) (drill 0.4) (layers "F.Cu" "B.Cu") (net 19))
 (segment (start 44.557591 122.318999) (end 43.528999 122.318999) (width 0.25) (layer "B.Cu") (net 19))
 (segment (start 72.5842 98.46399) (end 71.08101 98.46399) (width 0.25) (layer "B.Cu") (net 19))
 (segment (start 43.528999 122.318999) (end 42.943999 122.903999) (width 0.25) (layer "B.Cu") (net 19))
 (segment (start 42.943999 122.903999) (end 42.943999 123.984001) (width 0.25) (layer "B.Cu") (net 19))
 (segment (start 58.509001 119.163999) (end 59.309 118.364) (width 0.25) (layer "B.Cu") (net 19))
 (segment (start 77.978 92.964) (end 77.853 92.964) (width 0.25) (layer "B.Cu") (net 19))
 (segment (start 76.10501 94.94318) (end 72.5842 98.46399) (width 0.25) (layer "B.Cu") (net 19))
 (segment (start 43.528999 124.569001) (end 53.103999 124.569001) (width 0.25) (layer "B.Cu") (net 19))
 (segment (start 76.10501 94.71199) (end 76.10501 94.94318) (width 0.25) (layer "B.Cu") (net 19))
 (segment (start 71.08101 98.46399) (end 69.215 100.33) (width 0.25) (layer "B.Cu") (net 19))
 (segment (start 53.103999 124.569001) (end 58.509001 119.163999) (width 0.25) (layer "B.Cu") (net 19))
 (segment (start 57.004001 109.365999) (end 57.004001 109.872589) (width 0.25) (layer "B.Cu") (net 19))
 (segment (start 57.404 108.966) (end 57.004001 109.365999) (width 0.25) (layer "B.Cu") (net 19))
 (segment (start 57.004001 109.872589) (end 44.557591 122.318999) (width 0.25) (layer "B.Cu") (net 19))
 (segment (start 42.943999 123.984001) (end 43.528999 124.569001) (width 0.25) (layer "B.Cu") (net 19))
 (segment (start 77.853 92.964) (end 76.10501 94.71199) (width 0.25) (layer "B.Cu") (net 19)))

